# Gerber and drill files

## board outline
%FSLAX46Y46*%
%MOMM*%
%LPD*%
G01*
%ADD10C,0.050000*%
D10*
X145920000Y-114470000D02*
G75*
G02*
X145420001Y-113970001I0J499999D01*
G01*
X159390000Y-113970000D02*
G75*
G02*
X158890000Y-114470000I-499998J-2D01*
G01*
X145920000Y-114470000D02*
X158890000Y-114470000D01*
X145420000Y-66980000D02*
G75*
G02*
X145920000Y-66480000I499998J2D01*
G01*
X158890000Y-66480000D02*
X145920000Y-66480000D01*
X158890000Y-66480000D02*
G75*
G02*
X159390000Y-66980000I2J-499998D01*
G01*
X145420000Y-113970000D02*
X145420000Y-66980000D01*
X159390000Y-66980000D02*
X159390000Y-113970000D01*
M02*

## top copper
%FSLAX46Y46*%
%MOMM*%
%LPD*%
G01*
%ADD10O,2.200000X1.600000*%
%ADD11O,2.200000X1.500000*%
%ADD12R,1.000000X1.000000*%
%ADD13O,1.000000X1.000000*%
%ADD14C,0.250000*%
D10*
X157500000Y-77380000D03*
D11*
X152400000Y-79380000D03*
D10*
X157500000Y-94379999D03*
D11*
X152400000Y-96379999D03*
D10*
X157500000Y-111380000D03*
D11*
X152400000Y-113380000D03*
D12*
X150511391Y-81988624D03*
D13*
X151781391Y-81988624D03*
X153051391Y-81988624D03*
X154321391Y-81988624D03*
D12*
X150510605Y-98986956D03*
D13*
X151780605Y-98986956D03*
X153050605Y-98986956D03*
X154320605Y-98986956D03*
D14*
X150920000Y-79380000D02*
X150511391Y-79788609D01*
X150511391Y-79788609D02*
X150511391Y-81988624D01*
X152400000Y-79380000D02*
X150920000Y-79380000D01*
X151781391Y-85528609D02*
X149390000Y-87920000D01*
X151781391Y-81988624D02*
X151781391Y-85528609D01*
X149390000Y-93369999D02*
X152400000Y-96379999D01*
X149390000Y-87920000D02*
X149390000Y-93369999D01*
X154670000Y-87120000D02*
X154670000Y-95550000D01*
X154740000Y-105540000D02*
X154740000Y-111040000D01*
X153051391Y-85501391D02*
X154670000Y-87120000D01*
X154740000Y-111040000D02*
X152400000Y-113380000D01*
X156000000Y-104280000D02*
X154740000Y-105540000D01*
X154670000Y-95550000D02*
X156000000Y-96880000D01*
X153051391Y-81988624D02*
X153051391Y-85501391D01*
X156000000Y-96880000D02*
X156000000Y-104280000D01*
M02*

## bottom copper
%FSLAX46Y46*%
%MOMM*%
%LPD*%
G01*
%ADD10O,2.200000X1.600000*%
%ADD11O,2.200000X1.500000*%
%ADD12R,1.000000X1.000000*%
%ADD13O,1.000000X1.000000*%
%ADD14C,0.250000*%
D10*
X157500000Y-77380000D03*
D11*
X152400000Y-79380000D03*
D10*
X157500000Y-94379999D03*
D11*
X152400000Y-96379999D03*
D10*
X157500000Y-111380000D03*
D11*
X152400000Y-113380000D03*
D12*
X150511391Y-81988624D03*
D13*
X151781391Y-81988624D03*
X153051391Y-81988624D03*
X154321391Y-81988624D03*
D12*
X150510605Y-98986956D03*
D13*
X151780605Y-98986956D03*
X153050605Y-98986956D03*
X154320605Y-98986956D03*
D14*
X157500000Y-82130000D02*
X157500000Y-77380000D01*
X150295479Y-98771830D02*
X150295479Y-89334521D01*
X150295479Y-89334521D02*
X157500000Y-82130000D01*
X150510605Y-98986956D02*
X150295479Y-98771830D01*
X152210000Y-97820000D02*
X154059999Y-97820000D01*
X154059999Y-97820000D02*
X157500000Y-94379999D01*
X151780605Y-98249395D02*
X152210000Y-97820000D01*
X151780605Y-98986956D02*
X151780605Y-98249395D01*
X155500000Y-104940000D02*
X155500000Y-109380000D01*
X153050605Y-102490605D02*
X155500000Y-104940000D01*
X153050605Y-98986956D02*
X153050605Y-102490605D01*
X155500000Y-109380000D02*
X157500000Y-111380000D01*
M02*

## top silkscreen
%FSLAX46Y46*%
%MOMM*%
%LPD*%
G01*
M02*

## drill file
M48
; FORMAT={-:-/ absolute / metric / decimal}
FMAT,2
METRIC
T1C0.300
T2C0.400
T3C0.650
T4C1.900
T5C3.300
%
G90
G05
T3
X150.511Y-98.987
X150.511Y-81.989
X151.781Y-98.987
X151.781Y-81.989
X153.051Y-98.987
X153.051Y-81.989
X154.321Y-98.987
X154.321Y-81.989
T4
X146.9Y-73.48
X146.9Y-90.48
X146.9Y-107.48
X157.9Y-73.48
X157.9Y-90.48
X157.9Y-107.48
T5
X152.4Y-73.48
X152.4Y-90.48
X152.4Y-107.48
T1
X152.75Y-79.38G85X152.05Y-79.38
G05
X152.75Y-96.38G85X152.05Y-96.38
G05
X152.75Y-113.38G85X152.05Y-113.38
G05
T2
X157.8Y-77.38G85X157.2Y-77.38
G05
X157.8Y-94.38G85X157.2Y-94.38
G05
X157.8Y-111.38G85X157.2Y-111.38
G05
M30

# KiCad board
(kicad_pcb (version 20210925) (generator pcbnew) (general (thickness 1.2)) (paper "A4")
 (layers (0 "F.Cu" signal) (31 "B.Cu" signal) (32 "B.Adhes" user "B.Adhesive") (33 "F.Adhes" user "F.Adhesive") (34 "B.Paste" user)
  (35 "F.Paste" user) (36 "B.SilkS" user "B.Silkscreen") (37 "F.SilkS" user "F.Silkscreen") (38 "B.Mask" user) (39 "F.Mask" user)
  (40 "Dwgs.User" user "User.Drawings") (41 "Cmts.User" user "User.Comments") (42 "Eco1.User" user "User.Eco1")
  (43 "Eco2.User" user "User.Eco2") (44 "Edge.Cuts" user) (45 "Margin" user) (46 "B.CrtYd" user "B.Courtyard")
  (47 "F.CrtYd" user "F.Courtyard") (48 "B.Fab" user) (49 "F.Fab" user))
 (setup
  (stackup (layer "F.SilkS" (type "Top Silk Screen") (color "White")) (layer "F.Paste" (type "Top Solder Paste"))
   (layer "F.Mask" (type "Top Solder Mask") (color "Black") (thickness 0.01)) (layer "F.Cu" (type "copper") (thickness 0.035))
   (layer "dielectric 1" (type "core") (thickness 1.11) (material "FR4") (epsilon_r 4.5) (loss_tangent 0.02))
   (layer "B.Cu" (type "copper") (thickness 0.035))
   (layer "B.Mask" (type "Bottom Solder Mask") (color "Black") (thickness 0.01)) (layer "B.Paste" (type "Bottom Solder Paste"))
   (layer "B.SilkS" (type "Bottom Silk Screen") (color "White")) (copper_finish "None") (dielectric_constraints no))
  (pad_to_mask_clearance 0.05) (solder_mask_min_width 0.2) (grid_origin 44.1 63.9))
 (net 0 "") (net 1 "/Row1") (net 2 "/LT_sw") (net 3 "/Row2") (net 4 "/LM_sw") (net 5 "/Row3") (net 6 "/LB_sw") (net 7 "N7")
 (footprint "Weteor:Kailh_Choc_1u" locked (layer "B.Cu") (at 152.4 73.48 180)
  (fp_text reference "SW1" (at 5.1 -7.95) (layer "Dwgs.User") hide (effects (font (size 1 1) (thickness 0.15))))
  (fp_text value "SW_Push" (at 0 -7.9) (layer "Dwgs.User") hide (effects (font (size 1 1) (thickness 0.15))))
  (pad "" np_thru_hole circle locked (at 5.5 0 90) (size 1.9 1.9) (drill 1.9) (layers *.Cu *.Mask))
  (pad "" np_thru_hole circle locked (at 0 0 90) (size 3.3 3.3) (drill 3.3) (layers *.Cu *.Mask))
  (pad "" np_thru_hole circle locked (at -5.5 0 90) (size 1.9 1.9) (drill 1.9) (layers *.Cu *.Mask))
  (pad "1" thru_hole oval locked (at -5.1 -3.9 180) (size 2.2 1.6) (drill oval 1 0.4) (layers *.Cu "F.Mask") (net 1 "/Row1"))
  (pad "2" thru_hole oval locked (at 0 -5.9 180) (size 2.2 1.5) (drill oval 1 0.3) (layers *.Cu "F.Mask") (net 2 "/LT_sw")))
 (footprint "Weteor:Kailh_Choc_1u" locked (layer "B.Cu") (at 152.4 90.479999 180)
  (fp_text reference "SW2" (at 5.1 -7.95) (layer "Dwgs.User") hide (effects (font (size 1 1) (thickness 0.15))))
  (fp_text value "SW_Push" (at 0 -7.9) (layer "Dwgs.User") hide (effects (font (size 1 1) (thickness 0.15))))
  (pad "" np_thru_hole circle locked (at -5.5 0 90) (size 1.9 1.9) (drill 1.9) (layers *.Cu *.Mask))
  (pad "" np_thru_hole circle locked (at 0 0 90) (size 3.3 3.3) (drill 3.3) (layers *.Cu *.Mask))
  (pad "" np_thru_hole circle locked (at 5.5 0 90) (size 1.9 1.9) (drill 1.9) (layers *.Cu *.Mask))
  (pad "1" thru_hole oval locked (at -5.1 -3.9 180) (size 2.2 1.6) (drill oval 1 0.4) (layers *.Cu "F.Mask") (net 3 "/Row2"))
  (pad "2" thru_hole oval locked (at 0 -5.9 180) (size 2.2 1.5) (drill oval 1 0.3) (layers *.Cu "F.Mask") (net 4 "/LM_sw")))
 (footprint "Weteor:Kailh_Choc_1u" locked (layer "B.Cu") (at 152.4 107.48 180)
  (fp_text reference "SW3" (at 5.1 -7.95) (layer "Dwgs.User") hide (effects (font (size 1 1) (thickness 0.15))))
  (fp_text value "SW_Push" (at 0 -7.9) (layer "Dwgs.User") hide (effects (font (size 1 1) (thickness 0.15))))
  (pad "" np_thru_hole circle locked (at -5.5 0 90) (size 1.9 1.9) (drill 1.9) (layers *.Cu *.Mask))
  (pad "" np_thru_hole circle locked (at 0 0 90) (size 3.3 3.3) (drill 3.3) (layers *.Cu *.Mask))
  (pad "" np_thru_hole circle locked (at 5.5 0 90) (size 1.9 1.9) (drill 1.9) (layers *.Cu *.Mask))
  (pad "1" thru_hole oval locked (at -5.1 -3.9 180) (size 2.2 1.6) (drill oval 1 0.4) (layers *.Cu "F.Mask") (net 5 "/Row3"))
  (pad "2" thru_hole oval locked (at 0 -5.9 180) (size 2.2 1.5) (drill oval 1 0.3) (layers *.Cu "F.Mask") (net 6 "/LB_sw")))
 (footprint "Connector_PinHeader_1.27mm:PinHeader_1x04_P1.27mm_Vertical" (layer "B.Cu") (at 150.511391 81.988624 -90)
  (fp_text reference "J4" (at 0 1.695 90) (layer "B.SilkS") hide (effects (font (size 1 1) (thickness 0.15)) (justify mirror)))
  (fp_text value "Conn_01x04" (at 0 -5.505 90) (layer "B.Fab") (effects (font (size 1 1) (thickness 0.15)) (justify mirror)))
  (pad "1" thru_hole rect (at 0 0 270) (size 1 1) (drill 0.65) (layers *.Cu *.Mask) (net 2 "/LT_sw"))
  (pad "2" thru_hole oval (at 0 -1.27 270) (size 1 1) (drill 0.65) (layers *.Cu *.Mask) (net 4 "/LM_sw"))
  (pad "3" thru_hole oval (at 0 -2.54 270) (size 1 1) (drill 0.65) (layers *.Cu *.Mask) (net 6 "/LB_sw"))
  (pad "4" thru_hole oval (at 0 -3.81 270) (size 1 1) (drill 0.65) (layers *.Cu *.Mask)))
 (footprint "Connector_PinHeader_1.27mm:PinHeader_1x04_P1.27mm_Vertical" (layer "B.Cu") (at 150.510605 98.986956 -90)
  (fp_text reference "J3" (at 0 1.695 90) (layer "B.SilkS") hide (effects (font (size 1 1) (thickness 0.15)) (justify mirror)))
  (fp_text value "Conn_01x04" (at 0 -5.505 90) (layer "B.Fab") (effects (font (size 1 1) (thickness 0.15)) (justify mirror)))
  (pad "1" thru_hole rect (at 0 0 270) (size 1 1) (drill 0.65) (layers *.Cu *.Mask) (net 1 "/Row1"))
  (pad "2" thru_hole oval (at 0 -1.27 270) (size 1 1) (drill 0.65) (layers *.Cu *.Mask) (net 3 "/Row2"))
  (pad "3" thru_hole oval (at 0 -2.54 270) (size 1 1) (drill 0.65) (layers *.Cu *.Mask) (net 5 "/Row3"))
  (pad "4" thru_hole oval (at 0 -3.81 270) (size 1 1) (drill 0.65) (layers *.Cu *.Mask) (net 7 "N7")))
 (gr_arc (start 145.92 113.970001) (end 145.92 114.47) (angle 90) (layer "Edge.Cuts") (width 0.05))
 (gr_arc (start 158.890002 113.970002) (end 159.39 113.97) (angle 90.00045837) (layer "Edge.Cuts") (width 0.05))
 (gr_line (start 145.92 114.47) (end 158.89 114.47) (layer "Edge.Cuts") (width 0.05))
 (gr_arc (start 145.919998 66.979998) (end 145.42 66.98) (angle 90.00045837) (layer "Edge.Cuts") (width 0.05))
 (gr_line (start 158.89 66.48) (end 145.92 66.48) (layer "Edge.Cuts") (width 0.05))
 (gr_arc (start 158.890002 66.979998) (end 158.89 66.48) (angle 90.00045837) (layer "Edge.Cuts") (width 0.05))
 (gr_line (start 145.42 113.97) (end 145.42 66.98) (layer "Edge.Cuts") (width 0.05))
 (gr_line (start 159.39 66.98) (end 159.39 113.97) (layer "Edge.Cuts") (width 0.05))
 (segment (start 150.92 79.38) (end 150.511391 79.788609) (width 0.25) (layer "F.Cu") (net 2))
 (segment (start 150.511391 79.788609) (end 150.511391 81.988624) (width 0.25) (layer "F.Cu") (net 2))
 (segment (start 152.4 79.38) (end 150.92 79.38) (width 0.25) (layer "F.Cu") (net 2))
 (segment (start 151.781391 85.528609) (end 149.39 87.92) (width 0.25) (layer "F.Cu") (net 4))
 (segment (start 151.781391 81.988624) (end 151.781391 85.528609) (width 0.25) (layer "F.Cu") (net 4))
 (segment (start 149.39 93.369999) (end 152.4 96.379999) (width 0.25) (layer "F.Cu") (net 4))
 (segment (start 149.39 87.92) (end 149.39 93.369999) (width 0.25) (layer "F.Cu") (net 4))
 (segment (start 154.67 87.12) (end 154.67 95.55) (width 0.25) (layer "F.Cu") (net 6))
 (segment (start 154.74 105.54) (end 154.74 111.04) (width 0.25) (layer "F.Cu") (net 6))
 (segment (start 153.051391 85.501391) (end 154.67 87.12) (width 0.25) (layer "F.Cu") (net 6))
 (segment (start 154.74 111.04) (end 152.4 113.38) (width 0.25) (layer "F.Cu") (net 6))
 (segment (start 156 104.28) (end 154.74 105.54) (width 0.25) (layer "F.Cu") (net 6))
 (segment (start 154.67 95.55) (end 156 96.88) (width 0.25) (layer "F.Cu") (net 6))
 (segment (start 153.051391 81.988624) (end 153.051391 85.501391) (width 0.25) (layer "F.Cu") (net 6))
 (segment (start 156 96.88) (end 156 104.28) (width 0.25) (layer "F.Cu") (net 6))
 (segment (start 157.5 82.13) (end 157.5 77.38) (width 0.25) (layer "B.Cu") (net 1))
 (segment (start 150.295479 98.77183) (end 150.295479 89.334521) (width 0.25) (layer "B.Cu") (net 1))
 (segment (start 150.295479 89.334521) (end 157.5 82.13) (width 0.25) (layer "B.Cu") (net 1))
 (segment (start 150.510605 98.986956) (end 150.295479 98.77183) (width 0.25) (layer "B.Cu") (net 1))
 (segment (start 152.21 97.82) (end 154.059999 97.82) (width 0.25) (layer "B.Cu") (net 3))
 (segment (start 154.059999 97.82) (end 157.5 94.379999) (width 0.25) (layer "B.Cu") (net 3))
 (segment (start 151.780605 98.249395) (end 152.21 97.82) (width 0.25) (layer "B.Cu") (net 3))
 (segment (start 151.780605 98.986956) (end 151.780605 98.249395) (width 0.25) (layer "B.Cu") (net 3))
 (segment (start 155.5 104.94) (end 155.5 109.38) (width 0.25) (layer "B.Cu") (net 5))
 (segment (start 153.050605 102.490605) (end 155.5 104.94) (width 0.25) (layer "B.Cu") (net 5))
 (segment (start 153.050605 98.986956) (end 153.050605 102.490605) (width 0.25) (layer "B.Cu") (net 5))
 (segment (start 155.5 109.38) (end 157.5 111.38) (width 0.25) (layer "B.Cu") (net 5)))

